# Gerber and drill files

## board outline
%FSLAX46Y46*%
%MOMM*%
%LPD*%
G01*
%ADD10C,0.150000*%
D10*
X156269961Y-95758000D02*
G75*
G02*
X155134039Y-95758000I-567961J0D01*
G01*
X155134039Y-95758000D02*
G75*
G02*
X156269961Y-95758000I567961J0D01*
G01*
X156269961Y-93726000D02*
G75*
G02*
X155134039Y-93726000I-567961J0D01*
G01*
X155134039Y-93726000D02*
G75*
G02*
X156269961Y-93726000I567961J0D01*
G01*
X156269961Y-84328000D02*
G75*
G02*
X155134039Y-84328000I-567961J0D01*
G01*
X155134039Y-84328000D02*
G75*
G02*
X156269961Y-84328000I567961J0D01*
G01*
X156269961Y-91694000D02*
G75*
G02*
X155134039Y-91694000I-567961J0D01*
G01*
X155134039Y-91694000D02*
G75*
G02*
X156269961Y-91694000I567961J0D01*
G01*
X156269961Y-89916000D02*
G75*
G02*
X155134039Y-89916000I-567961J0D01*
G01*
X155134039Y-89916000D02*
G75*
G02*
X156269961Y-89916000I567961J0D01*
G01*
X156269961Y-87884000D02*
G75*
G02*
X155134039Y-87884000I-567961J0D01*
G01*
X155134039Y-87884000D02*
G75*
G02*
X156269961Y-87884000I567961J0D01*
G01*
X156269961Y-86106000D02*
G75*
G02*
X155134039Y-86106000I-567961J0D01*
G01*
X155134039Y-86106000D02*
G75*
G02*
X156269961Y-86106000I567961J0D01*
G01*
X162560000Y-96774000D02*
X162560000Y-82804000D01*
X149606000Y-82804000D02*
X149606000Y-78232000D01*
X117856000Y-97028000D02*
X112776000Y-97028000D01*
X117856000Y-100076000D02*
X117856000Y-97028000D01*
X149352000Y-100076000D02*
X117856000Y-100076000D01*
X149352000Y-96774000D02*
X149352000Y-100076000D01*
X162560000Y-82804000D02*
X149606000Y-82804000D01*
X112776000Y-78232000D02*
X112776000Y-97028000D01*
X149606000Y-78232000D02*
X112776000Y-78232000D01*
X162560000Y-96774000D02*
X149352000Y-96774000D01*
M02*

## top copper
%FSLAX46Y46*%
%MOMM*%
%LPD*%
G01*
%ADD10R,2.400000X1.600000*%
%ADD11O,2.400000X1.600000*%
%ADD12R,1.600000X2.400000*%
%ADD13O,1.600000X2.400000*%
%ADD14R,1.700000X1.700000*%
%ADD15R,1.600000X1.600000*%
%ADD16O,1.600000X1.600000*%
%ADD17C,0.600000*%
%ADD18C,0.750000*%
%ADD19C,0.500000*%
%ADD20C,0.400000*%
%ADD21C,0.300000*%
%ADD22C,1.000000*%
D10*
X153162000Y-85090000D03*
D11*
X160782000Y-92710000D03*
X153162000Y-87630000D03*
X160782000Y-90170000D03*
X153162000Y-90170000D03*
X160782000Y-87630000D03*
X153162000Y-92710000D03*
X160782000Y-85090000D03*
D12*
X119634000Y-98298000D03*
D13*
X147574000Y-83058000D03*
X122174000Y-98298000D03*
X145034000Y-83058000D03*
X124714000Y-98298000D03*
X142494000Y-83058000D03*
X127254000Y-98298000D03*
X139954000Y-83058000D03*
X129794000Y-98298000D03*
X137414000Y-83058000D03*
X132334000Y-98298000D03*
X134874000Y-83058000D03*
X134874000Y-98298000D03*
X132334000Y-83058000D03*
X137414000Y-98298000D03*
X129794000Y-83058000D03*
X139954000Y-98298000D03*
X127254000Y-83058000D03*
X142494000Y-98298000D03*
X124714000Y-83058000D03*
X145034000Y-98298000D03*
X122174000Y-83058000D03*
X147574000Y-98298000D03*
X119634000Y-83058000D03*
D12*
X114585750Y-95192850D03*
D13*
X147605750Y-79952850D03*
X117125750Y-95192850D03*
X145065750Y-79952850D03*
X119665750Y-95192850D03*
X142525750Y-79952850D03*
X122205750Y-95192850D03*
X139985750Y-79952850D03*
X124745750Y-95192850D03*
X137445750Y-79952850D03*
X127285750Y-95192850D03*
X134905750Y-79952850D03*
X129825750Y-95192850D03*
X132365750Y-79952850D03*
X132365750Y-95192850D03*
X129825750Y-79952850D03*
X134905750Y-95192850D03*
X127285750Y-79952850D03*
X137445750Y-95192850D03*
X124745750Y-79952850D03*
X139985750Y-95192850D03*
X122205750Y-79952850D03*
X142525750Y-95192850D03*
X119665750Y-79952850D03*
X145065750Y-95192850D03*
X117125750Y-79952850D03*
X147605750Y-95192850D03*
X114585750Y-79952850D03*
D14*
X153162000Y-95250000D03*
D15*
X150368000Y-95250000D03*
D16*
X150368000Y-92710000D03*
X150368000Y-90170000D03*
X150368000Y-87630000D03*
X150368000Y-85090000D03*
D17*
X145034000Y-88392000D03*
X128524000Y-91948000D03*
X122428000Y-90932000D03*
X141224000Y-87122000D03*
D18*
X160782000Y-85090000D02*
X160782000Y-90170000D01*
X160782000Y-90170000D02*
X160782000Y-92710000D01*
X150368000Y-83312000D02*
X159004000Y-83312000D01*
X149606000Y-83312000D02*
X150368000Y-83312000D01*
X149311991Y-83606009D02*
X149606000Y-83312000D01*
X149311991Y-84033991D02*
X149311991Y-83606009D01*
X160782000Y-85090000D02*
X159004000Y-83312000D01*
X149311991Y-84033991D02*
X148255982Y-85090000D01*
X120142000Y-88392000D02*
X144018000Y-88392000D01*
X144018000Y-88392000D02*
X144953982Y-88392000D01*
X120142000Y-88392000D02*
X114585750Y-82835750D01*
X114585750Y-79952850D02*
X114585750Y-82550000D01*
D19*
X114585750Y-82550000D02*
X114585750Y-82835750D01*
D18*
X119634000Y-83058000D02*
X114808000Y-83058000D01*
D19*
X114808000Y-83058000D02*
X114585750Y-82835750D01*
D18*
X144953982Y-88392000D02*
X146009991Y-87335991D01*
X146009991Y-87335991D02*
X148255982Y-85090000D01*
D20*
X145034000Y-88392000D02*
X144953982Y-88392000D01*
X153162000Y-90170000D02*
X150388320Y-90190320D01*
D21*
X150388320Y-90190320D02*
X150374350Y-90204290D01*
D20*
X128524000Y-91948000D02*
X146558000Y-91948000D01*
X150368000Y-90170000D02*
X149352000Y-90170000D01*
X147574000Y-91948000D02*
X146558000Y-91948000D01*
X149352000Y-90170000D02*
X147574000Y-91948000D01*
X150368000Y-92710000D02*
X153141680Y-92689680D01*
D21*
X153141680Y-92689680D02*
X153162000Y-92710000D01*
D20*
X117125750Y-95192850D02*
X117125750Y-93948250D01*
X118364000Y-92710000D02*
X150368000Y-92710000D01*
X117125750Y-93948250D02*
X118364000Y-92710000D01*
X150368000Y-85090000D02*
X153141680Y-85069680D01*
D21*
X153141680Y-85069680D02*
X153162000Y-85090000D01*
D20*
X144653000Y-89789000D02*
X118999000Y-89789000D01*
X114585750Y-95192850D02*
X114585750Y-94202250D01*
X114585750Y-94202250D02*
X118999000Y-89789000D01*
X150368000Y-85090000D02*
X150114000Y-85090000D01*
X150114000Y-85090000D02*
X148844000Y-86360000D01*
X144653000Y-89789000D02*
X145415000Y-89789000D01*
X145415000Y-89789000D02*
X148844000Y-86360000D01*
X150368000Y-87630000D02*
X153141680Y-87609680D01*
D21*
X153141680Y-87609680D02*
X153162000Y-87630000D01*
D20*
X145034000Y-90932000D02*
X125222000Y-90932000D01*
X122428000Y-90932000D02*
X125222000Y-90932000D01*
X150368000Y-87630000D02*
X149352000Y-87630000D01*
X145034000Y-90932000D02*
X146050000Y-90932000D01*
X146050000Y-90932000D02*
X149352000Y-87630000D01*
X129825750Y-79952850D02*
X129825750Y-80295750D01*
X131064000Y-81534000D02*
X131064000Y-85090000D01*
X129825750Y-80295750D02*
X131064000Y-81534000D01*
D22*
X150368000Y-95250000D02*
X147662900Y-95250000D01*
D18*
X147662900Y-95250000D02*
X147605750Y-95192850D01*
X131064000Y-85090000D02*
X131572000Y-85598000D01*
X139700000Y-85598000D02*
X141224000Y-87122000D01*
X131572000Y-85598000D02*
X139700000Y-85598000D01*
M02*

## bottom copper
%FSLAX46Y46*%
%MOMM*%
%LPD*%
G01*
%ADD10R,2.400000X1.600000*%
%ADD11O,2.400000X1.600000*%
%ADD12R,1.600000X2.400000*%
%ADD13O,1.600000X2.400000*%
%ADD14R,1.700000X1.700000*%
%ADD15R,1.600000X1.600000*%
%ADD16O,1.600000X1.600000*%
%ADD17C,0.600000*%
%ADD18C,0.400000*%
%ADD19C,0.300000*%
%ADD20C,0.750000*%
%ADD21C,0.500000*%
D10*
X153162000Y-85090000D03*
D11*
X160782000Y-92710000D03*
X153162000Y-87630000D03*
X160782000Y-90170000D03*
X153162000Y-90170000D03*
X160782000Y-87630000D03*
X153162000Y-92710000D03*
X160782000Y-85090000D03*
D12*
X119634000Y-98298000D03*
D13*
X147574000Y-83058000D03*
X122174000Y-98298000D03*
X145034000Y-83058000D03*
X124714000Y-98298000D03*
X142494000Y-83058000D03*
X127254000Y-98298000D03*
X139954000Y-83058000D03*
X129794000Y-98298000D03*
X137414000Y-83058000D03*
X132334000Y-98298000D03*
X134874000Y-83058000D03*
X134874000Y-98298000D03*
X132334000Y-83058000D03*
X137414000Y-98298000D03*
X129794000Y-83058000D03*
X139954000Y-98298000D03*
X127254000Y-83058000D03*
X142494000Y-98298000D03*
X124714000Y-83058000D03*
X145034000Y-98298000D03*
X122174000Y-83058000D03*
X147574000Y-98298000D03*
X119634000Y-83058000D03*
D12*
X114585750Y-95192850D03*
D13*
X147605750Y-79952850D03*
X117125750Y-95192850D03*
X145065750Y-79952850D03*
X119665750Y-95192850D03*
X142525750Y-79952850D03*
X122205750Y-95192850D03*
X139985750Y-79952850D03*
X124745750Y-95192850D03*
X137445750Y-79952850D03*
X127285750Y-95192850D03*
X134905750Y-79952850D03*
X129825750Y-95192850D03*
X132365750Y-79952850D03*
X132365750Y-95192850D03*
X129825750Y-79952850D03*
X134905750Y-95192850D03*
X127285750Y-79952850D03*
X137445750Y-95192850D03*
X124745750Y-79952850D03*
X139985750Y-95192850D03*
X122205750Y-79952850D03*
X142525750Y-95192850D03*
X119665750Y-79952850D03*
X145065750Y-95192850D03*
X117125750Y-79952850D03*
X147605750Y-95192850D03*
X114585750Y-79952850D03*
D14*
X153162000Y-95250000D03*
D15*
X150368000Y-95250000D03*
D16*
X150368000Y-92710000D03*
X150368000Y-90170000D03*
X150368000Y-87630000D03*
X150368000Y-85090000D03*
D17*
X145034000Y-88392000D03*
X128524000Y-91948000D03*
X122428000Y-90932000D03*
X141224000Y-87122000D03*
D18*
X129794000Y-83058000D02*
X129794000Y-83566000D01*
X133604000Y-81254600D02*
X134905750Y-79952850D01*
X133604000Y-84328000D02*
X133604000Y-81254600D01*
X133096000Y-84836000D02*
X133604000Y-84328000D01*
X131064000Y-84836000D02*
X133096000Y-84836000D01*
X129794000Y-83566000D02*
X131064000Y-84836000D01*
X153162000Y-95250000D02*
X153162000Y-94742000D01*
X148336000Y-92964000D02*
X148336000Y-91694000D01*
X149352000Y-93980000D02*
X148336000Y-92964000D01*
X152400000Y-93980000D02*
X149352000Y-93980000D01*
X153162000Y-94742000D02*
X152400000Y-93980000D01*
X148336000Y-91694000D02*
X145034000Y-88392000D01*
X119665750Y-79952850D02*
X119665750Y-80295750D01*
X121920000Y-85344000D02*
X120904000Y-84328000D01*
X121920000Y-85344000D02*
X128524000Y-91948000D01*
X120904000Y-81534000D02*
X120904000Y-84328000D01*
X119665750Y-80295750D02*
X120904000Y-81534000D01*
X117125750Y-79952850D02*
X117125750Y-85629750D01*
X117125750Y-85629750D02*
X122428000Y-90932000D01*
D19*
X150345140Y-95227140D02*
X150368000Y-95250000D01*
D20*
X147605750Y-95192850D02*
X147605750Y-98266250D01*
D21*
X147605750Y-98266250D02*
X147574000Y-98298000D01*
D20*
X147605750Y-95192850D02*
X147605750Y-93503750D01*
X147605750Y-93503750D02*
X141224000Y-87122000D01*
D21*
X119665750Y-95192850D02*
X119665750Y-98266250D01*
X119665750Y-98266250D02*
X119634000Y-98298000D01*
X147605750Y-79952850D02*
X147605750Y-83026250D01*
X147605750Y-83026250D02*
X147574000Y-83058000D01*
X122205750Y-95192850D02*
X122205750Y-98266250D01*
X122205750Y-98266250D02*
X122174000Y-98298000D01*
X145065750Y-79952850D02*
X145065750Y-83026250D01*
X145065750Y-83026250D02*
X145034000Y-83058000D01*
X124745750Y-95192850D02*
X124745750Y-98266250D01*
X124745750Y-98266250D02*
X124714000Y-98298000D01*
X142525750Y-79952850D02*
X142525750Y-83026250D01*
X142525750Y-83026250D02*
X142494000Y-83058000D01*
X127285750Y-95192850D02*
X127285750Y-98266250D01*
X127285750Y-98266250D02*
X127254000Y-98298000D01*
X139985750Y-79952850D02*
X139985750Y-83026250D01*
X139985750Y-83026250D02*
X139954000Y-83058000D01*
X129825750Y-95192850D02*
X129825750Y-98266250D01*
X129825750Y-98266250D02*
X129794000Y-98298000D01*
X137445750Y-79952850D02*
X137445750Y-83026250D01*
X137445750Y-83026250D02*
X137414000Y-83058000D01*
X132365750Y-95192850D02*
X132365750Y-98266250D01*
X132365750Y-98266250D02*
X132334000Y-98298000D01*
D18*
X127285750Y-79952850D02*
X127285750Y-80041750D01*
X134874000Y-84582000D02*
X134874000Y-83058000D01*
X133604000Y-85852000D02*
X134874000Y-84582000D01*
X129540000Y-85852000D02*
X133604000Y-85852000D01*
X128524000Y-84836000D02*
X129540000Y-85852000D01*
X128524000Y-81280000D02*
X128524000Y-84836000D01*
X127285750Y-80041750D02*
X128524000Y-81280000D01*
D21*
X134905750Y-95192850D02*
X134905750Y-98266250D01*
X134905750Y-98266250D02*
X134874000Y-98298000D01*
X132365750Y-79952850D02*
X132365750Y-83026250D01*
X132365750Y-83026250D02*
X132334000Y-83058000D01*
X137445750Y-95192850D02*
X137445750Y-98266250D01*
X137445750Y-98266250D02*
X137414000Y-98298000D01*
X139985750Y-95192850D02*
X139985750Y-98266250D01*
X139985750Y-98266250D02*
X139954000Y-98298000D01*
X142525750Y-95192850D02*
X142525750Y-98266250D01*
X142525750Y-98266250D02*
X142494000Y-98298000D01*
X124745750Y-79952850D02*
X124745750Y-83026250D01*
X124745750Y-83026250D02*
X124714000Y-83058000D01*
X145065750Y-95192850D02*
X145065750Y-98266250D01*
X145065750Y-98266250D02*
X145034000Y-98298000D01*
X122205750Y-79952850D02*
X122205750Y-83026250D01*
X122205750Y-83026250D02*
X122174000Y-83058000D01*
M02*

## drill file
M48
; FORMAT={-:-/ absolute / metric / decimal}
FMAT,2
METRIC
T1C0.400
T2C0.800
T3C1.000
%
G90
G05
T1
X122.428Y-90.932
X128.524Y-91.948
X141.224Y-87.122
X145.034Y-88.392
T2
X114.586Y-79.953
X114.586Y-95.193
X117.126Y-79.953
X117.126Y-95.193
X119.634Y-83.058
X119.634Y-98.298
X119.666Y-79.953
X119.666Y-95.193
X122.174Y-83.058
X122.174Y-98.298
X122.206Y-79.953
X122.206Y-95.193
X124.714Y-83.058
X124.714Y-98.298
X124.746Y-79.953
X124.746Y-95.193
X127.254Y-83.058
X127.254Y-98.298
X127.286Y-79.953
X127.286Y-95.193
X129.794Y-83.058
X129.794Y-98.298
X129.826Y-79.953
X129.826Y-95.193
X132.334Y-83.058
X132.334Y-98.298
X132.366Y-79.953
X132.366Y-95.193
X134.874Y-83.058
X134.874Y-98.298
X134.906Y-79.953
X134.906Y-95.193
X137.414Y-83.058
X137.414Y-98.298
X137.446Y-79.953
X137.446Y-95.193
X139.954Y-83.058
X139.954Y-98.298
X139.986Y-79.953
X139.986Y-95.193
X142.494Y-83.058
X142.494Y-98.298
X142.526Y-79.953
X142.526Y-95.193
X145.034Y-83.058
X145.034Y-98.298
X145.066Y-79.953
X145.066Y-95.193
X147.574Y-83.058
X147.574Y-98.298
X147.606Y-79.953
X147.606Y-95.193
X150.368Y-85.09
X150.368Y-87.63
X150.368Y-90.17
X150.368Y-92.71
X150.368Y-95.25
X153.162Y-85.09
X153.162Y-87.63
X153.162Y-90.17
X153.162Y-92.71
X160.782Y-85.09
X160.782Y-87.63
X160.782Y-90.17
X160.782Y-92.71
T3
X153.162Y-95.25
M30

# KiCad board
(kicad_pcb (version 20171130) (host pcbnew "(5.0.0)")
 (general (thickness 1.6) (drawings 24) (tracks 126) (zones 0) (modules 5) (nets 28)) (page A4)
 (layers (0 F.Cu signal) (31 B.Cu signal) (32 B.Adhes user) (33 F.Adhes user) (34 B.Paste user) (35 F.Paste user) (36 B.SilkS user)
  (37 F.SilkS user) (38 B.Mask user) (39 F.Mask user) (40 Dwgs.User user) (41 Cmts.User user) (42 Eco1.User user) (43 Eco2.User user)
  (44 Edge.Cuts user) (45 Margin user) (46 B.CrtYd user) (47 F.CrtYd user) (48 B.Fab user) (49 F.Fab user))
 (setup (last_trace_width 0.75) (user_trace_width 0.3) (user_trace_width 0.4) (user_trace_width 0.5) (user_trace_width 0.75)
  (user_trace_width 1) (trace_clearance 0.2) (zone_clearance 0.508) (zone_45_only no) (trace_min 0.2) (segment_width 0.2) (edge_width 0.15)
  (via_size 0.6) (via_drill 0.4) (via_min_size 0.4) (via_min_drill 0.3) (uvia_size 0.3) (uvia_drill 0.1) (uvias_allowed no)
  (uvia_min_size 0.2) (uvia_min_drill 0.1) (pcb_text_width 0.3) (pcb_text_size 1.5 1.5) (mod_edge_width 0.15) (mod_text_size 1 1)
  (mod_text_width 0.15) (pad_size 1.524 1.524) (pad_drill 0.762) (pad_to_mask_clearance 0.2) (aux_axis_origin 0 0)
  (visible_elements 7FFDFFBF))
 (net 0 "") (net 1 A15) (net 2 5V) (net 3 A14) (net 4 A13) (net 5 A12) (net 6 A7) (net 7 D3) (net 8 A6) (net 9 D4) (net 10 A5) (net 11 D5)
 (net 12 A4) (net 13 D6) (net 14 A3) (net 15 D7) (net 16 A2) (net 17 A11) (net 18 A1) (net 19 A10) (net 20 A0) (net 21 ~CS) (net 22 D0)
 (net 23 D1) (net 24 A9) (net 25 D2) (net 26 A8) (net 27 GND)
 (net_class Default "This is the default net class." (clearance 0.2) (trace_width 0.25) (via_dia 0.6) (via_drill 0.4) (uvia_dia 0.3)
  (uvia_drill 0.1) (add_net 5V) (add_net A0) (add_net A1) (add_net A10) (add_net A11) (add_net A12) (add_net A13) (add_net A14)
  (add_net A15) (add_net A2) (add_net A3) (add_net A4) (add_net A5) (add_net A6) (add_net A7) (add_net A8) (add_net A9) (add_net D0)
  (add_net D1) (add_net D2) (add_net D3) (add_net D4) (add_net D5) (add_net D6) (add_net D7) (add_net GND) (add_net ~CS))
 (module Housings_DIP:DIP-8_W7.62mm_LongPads (layer F.Cu) (at 153.162 85.09)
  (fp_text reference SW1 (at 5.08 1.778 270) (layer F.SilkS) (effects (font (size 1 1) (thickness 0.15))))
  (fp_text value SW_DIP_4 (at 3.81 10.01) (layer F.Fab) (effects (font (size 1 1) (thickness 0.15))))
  (pad 1 thru_hole rect (at 0 0) (size 2.4 1.6) (drill 0.8) (layers *.Cu *.Mask) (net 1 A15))
  (pad 5 thru_hole oval (at 7.62 7.62) (size 2.4 1.6) (drill 0.8) (layers *.Cu *.Mask) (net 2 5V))
  (pad 2 thru_hole oval (at 0 2.54) (size 2.4 1.6) (drill 0.8) (layers *.Cu *.Mask) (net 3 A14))
  (pad 6 thru_hole oval (at 7.62 5.08) (size 2.4 1.6) (drill 0.8) (layers *.Cu *.Mask) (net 2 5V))
  (pad 3 thru_hole oval (at 0 5.08) (size 2.4 1.6) (drill 0.8) (layers *.Cu *.Mask) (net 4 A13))
  (pad 7 thru_hole oval (at 7.62 2.54) (size 2.4 1.6) (drill 0.8) (layers *.Cu *.Mask) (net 2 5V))
  (pad 4 thru_hole oval (at 0 7.62) (size 2.4 1.6) (drill 0.8) (layers *.Cu *.Mask) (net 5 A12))
  (pad 8 thru_hole oval (at 7.62 0) (size 2.4 1.6) (drill 0.8) (layers *.Cu *.Mask) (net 2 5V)))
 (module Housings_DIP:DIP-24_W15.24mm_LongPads (layer F.Cu) (at 119.634 98.298 90)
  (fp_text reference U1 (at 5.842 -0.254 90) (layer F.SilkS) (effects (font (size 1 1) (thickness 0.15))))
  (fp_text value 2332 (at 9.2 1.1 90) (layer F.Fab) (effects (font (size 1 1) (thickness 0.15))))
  (pad 1 thru_hole rect (at 0 0 90) (size 2.4 1.6) (drill 0.8) (layers *.Cu *.Mask) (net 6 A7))
  (pad 13 thru_hole oval (at 15.24 27.94 90) (size 2.4 1.6) (drill 0.8) (layers *.Cu *.Mask) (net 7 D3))
  (pad 2 thru_hole oval (at 0 2.54 90) (size 2.4 1.6) (drill 0.8) (layers *.Cu *.Mask) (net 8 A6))
  (pad 14 thru_hole oval (at 15.24 25.4 90) (size 2.4 1.6) (drill 0.8) (layers *.Cu *.Mask) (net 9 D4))
  (pad 3 thru_hole oval (at 0 5.08 90) (size 2.4 1.6) (drill 0.8) (layers *.Cu *.Mask) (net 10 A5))
  (pad 15 thru_hole oval (at 15.24 22.86 90) (size 2.4 1.6) (drill 0.8) (layers *.Cu *.Mask) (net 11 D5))
  (pad 4 thru_hole oval (at 0 7.62 90) (size 2.4 1.6) (drill 0.8) (layers *.Cu *.Mask) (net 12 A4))
  (pad 16 thru_hole oval (at 15.24 20.32 90) (size 2.4 1.6) (drill 0.8) (layers *.Cu *.Mask) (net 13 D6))
  (pad 5 thru_hole oval (at 0 10.16 90) (size 2.4 1.6) (drill 0.8) (layers *.Cu *.Mask) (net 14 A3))
  (pad 17 thru_hole oval (at 15.24 17.78 90) (size 2.4 1.6) (drill 0.8) (layers *.Cu *.Mask) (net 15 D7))
  (pad 6 thru_hole oval (at 0 12.7 90) (size 2.4 1.6) (drill 0.8) (layers *.Cu *.Mask) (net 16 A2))
  (pad 18 thru_hole oval (at 15.24 15.24 90) (size 2.4 1.6) (drill 0.8) (layers *.Cu *.Mask) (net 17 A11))
  (pad 7 thru_hole oval (at 0 15.24 90) (size 2.4 1.6) (drill 0.8) (layers *.Cu *.Mask) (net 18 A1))
  (pad 19 thru_hole oval (at 15.24 12.7 90) (size 2.4 1.6) (drill 0.8) (layers *.Cu *.Mask) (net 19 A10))
  (pad 8 thru_hole oval (at 0 17.78 90) (size 2.4 1.6) (drill 0.8) (layers *.Cu *.Mask) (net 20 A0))
  (pad 20 thru_hole oval (at 15.24 10.16 90) (size 2.4 1.6) (drill 0.8) (layers *.Cu *.Mask) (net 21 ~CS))
  (pad 9 thru_hole oval (at 0 20.32 90) (size 2.4 1.6) (drill 0.8) (layers *.Cu *.Mask) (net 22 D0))
  (pad 21 thru_hole oval (at 15.24 7.62 90) (size 2.4 1.6) (drill 0.8) (layers *.Cu *.Mask))
  (pad 10 thru_hole oval (at 0 22.86 90) (size 2.4 1.6) (drill 0.8) (layers *.Cu *.Mask) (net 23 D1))
  (pad 22 thru_hole oval (at 15.24 5.08 90) (size 2.4 1.6) (drill 0.8) (layers *.Cu *.Mask) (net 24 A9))
  (pad 11 thru_hole oval (at 0 25.4 90) (size 2.4 1.6) (drill 0.8) (layers *.Cu *.Mask) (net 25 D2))
  (pad 23 thru_hole oval (at 15.24 2.54 90) (size 2.4 1.6) (drill 0.8) (layers *.Cu *.Mask) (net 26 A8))
  (pad 12 thru_hole oval (at 0 27.94 90) (size 2.4 1.6) (drill 0.8) (layers *.Cu *.Mask) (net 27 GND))
  (pad 24 thru_hole oval (at 15.24 0 90) (size 2.4 1.6) (drill 0.8) (layers *.Cu *.Mask) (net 2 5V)))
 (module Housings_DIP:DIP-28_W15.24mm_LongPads (layer F.Cu) (at 114.58575 95.19285 90)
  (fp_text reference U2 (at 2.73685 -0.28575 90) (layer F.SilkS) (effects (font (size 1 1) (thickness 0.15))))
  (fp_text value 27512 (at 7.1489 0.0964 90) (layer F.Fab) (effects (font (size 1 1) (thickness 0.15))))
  (pad 1 thru_hole rect (at 0 0 90) (size 2.4 1.6) (drill 0.8) (layers *.Cu *.Mask) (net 1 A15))
  (pad 15 thru_hole oval (at 15.24 33.02 90) (size 2.4 1.6) (drill 0.8) (layers *.Cu *.Mask) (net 7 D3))
  (pad 2 thru_hole oval (at 0 2.54 90) (size 2.4 1.6) (drill 0.8) (layers *.Cu *.Mask) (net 5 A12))
  (pad 16 thru_hole oval (at 15.24 30.48 90) (size 2.4 1.6) (drill 0.8) (layers *.Cu *.Mask) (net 9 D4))
  (pad 3 thru_hole oval (at 0 5.08 90) (size 2.4 1.6) (drill 0.8) (layers *.Cu *.Mask) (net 6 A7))
  (pad 17 thru_hole oval (at 15.24 27.94 90) (size 2.4 1.6) (drill 0.8) (layers *.Cu *.Mask) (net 11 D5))
  (pad 4 thru_hole oval (at 0 7.62 90) (size 2.4 1.6) (drill 0.8) (layers *.Cu *.Mask) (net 8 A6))
  (pad 18 thru_hole oval (at 15.24 25.4 90) (size 2.4 1.6) (drill 0.8) (layers *.Cu *.Mask) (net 13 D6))
  (pad 5 thru_hole oval (at 0 10.16 90) (size 2.4 1.6) (drill 0.8) (layers *.Cu *.Mask) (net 10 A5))
  (pad 19 thru_hole oval (at 15.24 22.86 90) (size 2.4 1.6) (drill 0.8) (layers *.Cu *.Mask) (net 15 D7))
  (pad 6 thru_hole oval (at 0 12.7 90) (size 2.4 1.6) (drill 0.8) (layers *.Cu *.Mask) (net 12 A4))
  (pad 20 thru_hole oval (at 15.24 20.32 90) (size 2.4 1.6) (drill 0.8) (layers *.Cu *.Mask) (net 21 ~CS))
  (pad 7 thru_hole oval (at 0 15.24 90) (size 2.4 1.6) (drill 0.8) (layers *.Cu *.Mask) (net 14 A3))
  (pad 21 thru_hole oval (at 15.24 17.78 90) (size 2.4 1.6) (drill 0.8) (layers *.Cu *.Mask) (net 19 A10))
  (pad 8 thru_hole oval (at 0 17.78 90) (size 2.4 1.6) (drill 0.8) (layers *.Cu *.Mask) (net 16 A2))
  (pad 22 thru_hole oval (at 15.24 15.24 90) (size 2.4 1.6) (drill 0.8) (layers *.Cu *.Mask) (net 27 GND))
  (pad 9 thru_hole oval (at 0 20.32 90) (size 2.4 1.6) (drill 0.8) (layers *.Cu *.Mask) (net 18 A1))
  (pad 23 thru_hole oval (at 15.24 12.7 90) (size 2.4 1.6) (drill 0.8) (layers *.Cu *.Mask) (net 17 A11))
  (pad 10 thru_hole oval (at 0 22.86 90) (size 2.4 1.6) (drill 0.8) (layers *.Cu *.Mask) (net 20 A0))
  (pad 24 thru_hole oval (at 15.24 10.16 90) (size 2.4 1.6) (drill 0.8) (layers *.Cu *.Mask) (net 24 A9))
  (pad 11 thru_hole oval (at 0 25.4 90) (size 2.4 1.6) (drill 0.8) (layers *.Cu *.Mask) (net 22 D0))
  (pad 25 thru_hole oval (at 15.24 7.62 90) (size 2.4 1.6) (drill 0.8) (layers *.Cu *.Mask) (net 26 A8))
  (pad 12 thru_hole oval (at 0 27.94 90) (size 2.4 1.6) (drill 0.8) (layers *.Cu *.Mask) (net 23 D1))
  (pad 26 thru_hole oval (at 15.24 5.08 90) (size 2.4 1.6) (drill 0.8) (layers *.Cu *.Mask) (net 4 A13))
  (pad 13 thru_hole oval (at 0 30.48 90) (size 2.4 1.6) (drill 0.8) (layers *.Cu *.Mask) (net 25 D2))
  (pad 27 thru_hole oval (at 15.24 2.54 90) (size 2.4 1.6) (drill 0.8) (layers *.Cu *.Mask) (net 3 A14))
  (pad 14 thru_hole oval (at 0 33.02 90) (size 2.4 1.6) (drill 0.8) (layers *.Cu *.Mask) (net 27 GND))
  (pad 28 thru_hole oval (at 15.24 0 90) (size 2.4 1.6) (drill 0.8) (layers *.Cu *.Mask) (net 2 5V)))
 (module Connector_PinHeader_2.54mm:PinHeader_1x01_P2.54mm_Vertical (layer F.Cu) (at 153.162 95.25 90)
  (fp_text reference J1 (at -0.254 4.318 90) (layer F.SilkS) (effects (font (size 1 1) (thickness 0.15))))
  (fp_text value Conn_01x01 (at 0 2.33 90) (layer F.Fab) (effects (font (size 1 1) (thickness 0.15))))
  (pad 1 thru_hole rect (at 0 0 90) (size 1.7 1.7) (drill 1) (layers *.Cu *.Mask) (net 2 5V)))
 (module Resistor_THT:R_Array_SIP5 (layer F.Cu) (at 150.368 95.25 90)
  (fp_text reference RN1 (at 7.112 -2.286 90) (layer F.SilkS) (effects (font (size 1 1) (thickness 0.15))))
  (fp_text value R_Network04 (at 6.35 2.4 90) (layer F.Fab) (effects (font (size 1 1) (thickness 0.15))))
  (pad 1 thru_hole rect (at 0 0 90) (size 1.6 1.6) (drill 0.8) (layers *.Cu *.Mask) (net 27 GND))
  (pad 2 thru_hole oval (at 2.54 0 90) (size 1.6 1.6) (drill 0.8) (layers *.Cu *.Mask) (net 5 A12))
  (pad 3 thru_hole oval (at 5.08 0 90) (size 1.6 1.6) (drill 0.8) (layers *.Cu *.Mask) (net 4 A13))
  (pad 4 thru_hole oval (at 7.62 0 90) (size 1.6 1.6) (drill 0.8) (layers *.Cu *.Mask) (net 3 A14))
  (pad 5 thru_hole oval (at 10.16 0 90) (size 1.6 1.6) (drill 0.8) (layers *.Cu *.Mask) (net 1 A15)))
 (gr_circle (center 155.702 95.758) (end 156.21 96.012) (layer Edge.Cuts) (width 0.15))
 (gr_circle (center 155.702 93.726) (end 156.21 93.98) (layer Edge.Cuts) (width 0.15))
 (gr_circle (center 155.702 84.328) (end 156.21 84.582) (layer Edge.Cuts) (width 0.15))
 (gr_circle (center 155.702 91.694) (end 155.956 92.202) (layer Edge.Cuts) (width 0.15))
 (gr_circle (center 155.702 89.916) (end 156.21 90.17) (layer Edge.Cuts) (width 0.15))
 (gr_circle (center 155.702 87.884) (end 156.21 88.138) (layer Edge.Cuts) (width 0.15))
 (gr_circle (center 155.702 86.106) (end 156.21 86.36) (layer Edge.Cuts) (width 0.15))
 (gr_line (start 162.56 96.774) (end 162.56 82.804) (angle 90) (layer Edge.Cuts) (width 0.15))
 (gr_line (start 149.606 82.804) (end 149.606 78.232) (angle 90) (layer Edge.Cuts) (width 0.15))
 (gr_line (start 117.856 97.028) (end 112.776 97.028) (angle 90) (layer Edge.Cuts) (width 0.15))
 (gr_line (start 117.856 100.076) (end 117.856 97.028) (angle 90) (layer Edge.Cuts) (width 0.15))
 (gr_line (start 149.352 100.076) (end 117.856 100.076) (angle 90) (layer Edge.Cuts) (width 0.15))
 (gr_line (start 149.352 96.774) (end 149.352 100.076) (angle 90) (layer Edge.Cuts) (width 0.15))
 (gr_line (start 162.56 82.804) (end 149.606 82.804) (angle 90) (layer Edge.Cuts) (width 0.15))
 (gr_line (start 112.776 78.232) (end 112.776 97.028) (angle 90) (layer Edge.Cuts) (width 0.15))
 (gr_line (start 149.606 78.232) (end 112.776 78.232) (angle 90) (layer Edge.Cuts) (width 0.15))
 (gr_line (start 162.56 96.774) (end 149.352 96.774) (angle 90) (layer Edge.Cuts) (width 0.15))
 (segment (start 129.794 83.058) (end 129.794 83.566) (width 0.4) (layer B.Cu) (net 21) (status C00000))
 (segment (start 133.604 81.2546) (end 134.90575 79.95285) (width 0.4) (layer B.Cu) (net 21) (status 800000))
 (segment (start 133.604 84.328) (end 133.604 81.2546) (width 0.4) (layer B.Cu) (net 21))
 (segment (start 133.096 84.836) (end 133.604 84.328) (width 0.4) (layer B.Cu) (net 21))
 (segment (start 131.064 84.836) (end 133.096 84.836) (width 0.4) (layer B.Cu) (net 21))
 (segment (start 129.794 83.566) (end 131.064 84.836) (width 0.4) (layer B.Cu) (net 21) (status 400000))
 (segment (start 160.782 85.09) (end 160.782 90.17) (width 0.75) (layer F.Cu) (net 2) (status C00030))
 (segment (start 160.782 90.17) (end 160.782 92.71) (width 0.75) (layer F.Cu) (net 2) (status C00030))
 (segment (start 150.368 83.312) (end 159.004 83.312) (width 0.75) (layer F.Cu) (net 2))
 (segment (start 149.606 83.312) (end 150.368 83.312) (width 0.75) (layer F.Cu) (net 2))
 (segment (start 149.311991 83.606009) (end 149.606 83.312) (width 0.75) (layer F.Cu) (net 2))
 (segment (start 149.311991 84.033991) (end 149.311991 83.606009) (width 0.75) (layer F.Cu) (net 2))
 (segment (start 160.782 85.09) (end 159.004 83.312) (width 0.75) (layer F.Cu) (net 2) (status 400000))
 (segment (start 149.311991 84.033991) (end 148.255982 85.09) (width 0.75) (layer F.Cu) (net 2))
 (segment (start 120.142 88.392) (end 144.018 88.392) (width 0.75) (layer F.Cu) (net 2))
 (segment (start 144.018 88.392) (end 144.953982 88.392) (width 0.75) (layer F.Cu) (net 2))
 (segment (start 120.142 88.392) (end 114.58575 82.83575) (width 0.75) (layer F.Cu) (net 2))
 (segment (start 114.58575 79.95285) (end 114.58575 82.55) (width 0.75) (layer F.Cu) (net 2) (status 400000))
 (segment (start 114.58575 82.55) (end 114.58575 82.83575) (width 0.5) (layer F.Cu) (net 2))
 (segment (start 119.634 83.058) (end 114.808 83.058) (width 0.75) (layer F.Cu) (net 2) (status 400000))
 (segment (start 114.808 83.058) (end 114.58575 82.83575) (width 0.5) (layer F.Cu) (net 2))
 (segment (start 144.953982 88.392) (end 146.009991 87.335991) (width 0.75) (layer F.Cu) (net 2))
 (segment (start 146.009991 87.335991) (end 148.255982 85.09) (width 0.75) (layer F.Cu) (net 2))
 (segment (start 153.162 95.25) (end 153.162 94.742) (width 0.4) (layer B.Cu) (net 2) (status C00000))
 (segment (start 148.336 92.964) (end 148.336 91.694) (width 0.4) (layer B.Cu) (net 2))
 (segment (start 149.352 93.98) (end 148.336 92.964) (width 0.4) (layer B.Cu) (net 2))
 (segment (start 152.4 93.98) (end 149.352 93.98) (width 0.4) (layer B.Cu) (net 2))
 (segment (start 153.162 94.742) (end 152.4 93.98) (width 0.4) (layer B.Cu) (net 2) (status 400000))
 (segment (start 148.336 91.694) (end 145.034 88.392) (width 0.4) (layer B.Cu) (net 2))
 (segment (start 145.034 88.392) (end 144.953982 88.392) (width 0.4) (layer F.Cu) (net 2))
 (via (at 145.034 88.392) (size 0.6) (drill 0.4) (layers F.Cu B.Cu) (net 2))
 (segment (start 153.162 90.17) (end 150.38832 90.19032) (width 0.4) (layer F.Cu) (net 4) (status C00010))
 (segment (start 150.38832 90.19032) (end 150.37435 90.20429) (width 0.3) (layer F.Cu) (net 4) (status C00030))
 (segment (start 119.66575 79.95285) (end 119.66575 80.29575) (width 0.4) (layer B.Cu) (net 4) (status C00000))
 (segment (start 121.92 85.344) (end 120.904 84.328) (width 0.4) (layer B.Cu) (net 4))
 (segment (start 121.92 85.344) (end 128.524 91.948) (width 0.4) (layer B.Cu) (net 4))
 (via (at 128.524 91.948) (size 0.6) (drill 0.4) (layers F.Cu B.Cu) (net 4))
 (segment (start 128.524 91.948) (end 146.558 91.948) (width 0.4) (layer F.Cu) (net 4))
 (segment (start 120.904 81.534) (end 120.904 84.328) (width 0.4) (layer B.Cu) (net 4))
 (segment (start 119.66575 80.29575) (end 120.904 81.534) (width 0.4) (layer B.Cu) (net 4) (status 400000))
 (segment (start 150.368 90.17) (end 149.352 90.17) (width 0.4) (layer F.Cu) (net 4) (status 400000))
 (segment (start 147.574 91.948) (end 146.558 91.948) (width 0.4) (layer F.Cu) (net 4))
 (segment (start 149.352 90.17) (end 147.574 91.948) (width 0.4) (layer F.Cu) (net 4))
 (segment (start 150.368 92.71) (end 153.14168 92.68968) (width 0.4) (layer F.Cu) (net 5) (status C00020))
 (segment (start 153.14168 92.68968) (end 153.162 92.71) (width 0.3) (layer F.Cu) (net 5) (status C00030))
 (segment (start 117.12575 95.19285) (end 117.12575 93.94825) (width 0.4) (layer F.Cu) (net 5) (status 400000))
 (segment (start 118.364 92.71) (end 150.368 92.71) (width 0.4) (layer F.Cu) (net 5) (status 800000))
 (segment (start 117.12575 93.94825) (end 118.364 92.71) (width 0.4) (layer F.Cu) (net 5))
 (segment (start 150.368 85.09) (end 153.14168 85.06968) (width 0.4) (layer F.Cu) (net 1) (status C00020))
 (segment (start 153.14168 85.06968) (end 153.162 85.09) (width 0.3) (layer F.Cu) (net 1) (status C00030))
 (segment (start 144.653 89.789) (end 118.999 89.789) (width 0.4) (layer F.Cu) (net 1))
 (segment (start 114.58575 95.19285) (end 114.58575 94.20225) (width 0.4) (layer F.Cu) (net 1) (status C00000))
 (segment (start 114.58575 94.20225) (end 118.999 89.789) (width 0.4) (layer F.Cu) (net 1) (status 400000))
 (segment (start 150.368 85.09) (end 150.114 85.09) (width 0.4) (layer F.Cu) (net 1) (status C00000))
 (segment (start 150.114 85.09) (end 148.844 86.36) (width 0.4) (layer F.Cu) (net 1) (status 400000))
 (segment (start 144.653 89.789) (end 145.415 89.789) (width 0.4) (layer F.Cu) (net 1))
 (segment (start 145.415 89.789) (end 148.844 86.36) (width 0.4) (layer F.Cu) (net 1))
 (segment (start 150.368 87.63) (end 153.14168 87.60968) (width 0.4) (layer F.Cu) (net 3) (status C00020))
 (segment (start 153.14168 87.60968) (end 153.162 87.63) (width 0.3) (layer F.Cu) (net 3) (status C00030))
 (segment (start 145.034 90.932) (end 125.222 90.932) (width 0.4) (layer F.Cu) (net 3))
 (segment (start 117.12575 79.95285) (end 117.12575 85.62975) (width 0.4) (layer B.Cu) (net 3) (status 400000))
 (segment (start 122.428 90.932) (end 125.222 90.932) (width 0.4) (layer F.Cu) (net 3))
 (via (at 122.428 90.932) (size 0.6) (drill 0.4) (layers F.Cu B.Cu) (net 3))
 (segment (start 117.12575 85.62975) (end 122.428 90.932) (width 0.4) (layer B.Cu) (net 3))
 (segment (start 150.368 87.63) (end 149.352 87.63) (width 0.4) (layer F.Cu) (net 3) (status 400000))
 (segment (start 145.034 90.932) (end 146.05 90.932) (width 0.4) (layer F.Cu) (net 3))
 (segment (start 146.05 90.932) (end 149.352 87.63) (width 0.4) (layer F.Cu) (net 3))
 (segment (start 150.34514 95.22714) (end 150.368 95.25) (width 0.3) (layer B.Cu) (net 27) (status C00030))
 (segment (start 147.60575 95.19285) (end 147.60575 98.26625) (width 0.75) (layer B.Cu) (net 27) (status C00000))
 (segment (start 147.60575 98.26625) (end 147.574 98.298) (width 0.5) (layer B.Cu) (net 27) (status C00000))
 (segment (start 129.82575 79.95285) (end 129.82575 80.29575) (width 0.4) (layer F.Cu) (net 27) (status C00000))
 (segment (start 131.064 81.534) (end 131.064 85.09) (width 0.4) (layer F.Cu) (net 27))
 (segment (start 129.82575 80.29575) (end 131.064 81.534) (width 0.4) (layer F.Cu) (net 27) (status 400000))
 (segment (start 150.368 95.25) (end 147.6629 95.25) (width 1) (layer F.Cu) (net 27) (status C00000))
 (segment (start 147.6629 95.25) (end 147.60575 95.19285) (width 0.75) (layer F.Cu) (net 27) (status C00000))
 (segment (start 147.60575 95.19285) (end 147.60575 93.50375) (width 0.75) (layer B.Cu) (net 27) (status 400000))
 (via (at 141.224 87.122) (size 0.6) (drill 0.4) (layers F.Cu B.Cu) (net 27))
 (segment (start 147.60575 93.50375) (end 141.224 87.122) (width 0.75) (layer B.Cu) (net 27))
 (segment (start 131.064 85.09) (end 131.572 85.598) (width 0.75) (layer F.Cu) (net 27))
 (segment (start 139.7 85.598) (end 141.224 87.122) (width 0.75) (layer F.Cu) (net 27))
 (segment (start 131.572 85.598) (end 139.7 85.598) (width 0.75) (layer F.Cu) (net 27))
 (segment (start 119.66575 95.19285) (end 119.66575 98.26625) (width 0.5) (layer B.Cu) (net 6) (status C00000))
 (segment (start 119.66575 98.26625) (end 119.634 98.298) (width 0.5) (layer B.Cu) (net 6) (status C00000))
 (segment (start 147.60575 79.95285) (end 147.60575 83.02625) (width 0.5) (layer B.Cu) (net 7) (status C00000))
 (segment (start 147.60575 83.02625) (end 147.574 83.058) (width 0.5) (layer B.Cu) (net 7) (status C00000))
 (segment (start 122.20575 95.19285) (end 122.20575 98.26625) (width 0.5) (layer B.Cu) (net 8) (status C00000))
 (segment (start 122.20575 98.26625) (end 122.174 98.298) (width 0.5) (layer B.Cu) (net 8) (status C00000))
 (segment (start 145.06575 79.95285) (end 145.06575 83.02625) (width 0.5) (layer B.Cu) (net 9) (status C00000))
 (segment (start 145.06575 83.02625) (end 145.034 83.058) (width 0.5) (layer B.Cu) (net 9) (status C00000))
 (segment (start 124.74575 95.19285) (end 124.74575 98.26625) (width 0.5) (layer B.Cu) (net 10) (status C00000))
 (segment (start 124.74575 98.26625) (end 124.714 98.298) (width 0.5) (layer B.Cu) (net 10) (status C00000))
 (segment (start 142.52575 79.95285) (end 142.52575 83.02625) (width 0.5) (layer B.Cu) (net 11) (status C00000))
 (segment (start 142.52575 83.02625) (end 142.494 83.058) (width 0.5) (layer B.Cu) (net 11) (status C00000))
 (segment (start 127.28575 95.19285) (end 127.28575 98.26625) (width 0.5) (layer B.Cu) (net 12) (status C00000))
 (segment (start 127.28575 98.26625) (end 127.254 98.298) (width 0.5) (layer B.Cu) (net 12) (status C00000))
 (segment (start 139.98575 79.95285) (end 139.98575 83.02625) (width 0.5) (layer B.Cu) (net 13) (status C00000))
 (segment (start 139.98575 83.02625) (end 139.954 83.058) (width 0.5) (layer B.Cu) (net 13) (status C00000))
 (segment (start 129.82575 95.19285) (end 129.82575 98.26625) (width 0.5) (layer B.Cu) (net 14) (status C00000))
 (segment (start 129.82575 98.26625) (end 129.794 98.298) (width 0.5) (layer B.Cu) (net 14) (status C00000))
 (segment (start 137.44575 79.95285) (end 137.44575 83.02625) (width 0.5) (layer B.Cu) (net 15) (status C00000))
 (segment (start 137.44575 83.02625) (end 137.414 83.058) (width 0.5) (layer B.Cu) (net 15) (status C00000))
 (segment (start 132.36575 95.19285) (end 132.36575 98.26625) (width 0.5) (layer B.Cu) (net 16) (status C00000))
 (segment (start 132.36575 98.26625) (end 132.334 98.298) (width 0.5) (layer B.Cu) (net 16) (status C00000))
 (segment (start 127.28575 79.95285) (end 127.28575 80.04175) (width 0.4) (layer B.Cu) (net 17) (status C00000))
 (segment (start 134.874 84.582) (end 134.874 83.058) (width 0.4) (layer B.Cu) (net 17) (status 800000))
 (segment (start 133.604 85.852) (end 134.874 84.582) (width 0.4) (layer B.Cu) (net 17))
 (segment (start 129.54 85.852) (end 133.604 85.852) (width 0.4) (layer B.Cu) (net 17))
 (segment (start 128.524 84.836) (end 129.54 85.852) (width 0.4) (layer B.Cu) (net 17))
 (segment (start 128.524 81.28) (end 128.524 84.836) (width 0.4) (layer B.Cu) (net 17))
 (segment (start 127.28575 80.04175) (end 128.524 81.28) (width 0.4) (layer B.Cu) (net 17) (status 400000))
 (segment (start 134.90575 95.19285) (end 134.90575 98.26625) (width 0.5) (layer B.Cu) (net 18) (status C00000))
 (segment (start 134.90575 98.26625) (end 134.874 98.298) (width 0.5) (layer B.Cu) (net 18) (status C00000))
 (segment (start 132.36575 79.95285) (end 132.36575 83.02625) (width 0.5) (layer B.Cu) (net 19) (status C00000))
 (segment (start 132.36575 83.02625) (end 132.334 83.058) (width 0.5) (layer B.Cu) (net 19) (status C00000))
 (segment (start 137.44575 95.19285) (end 137.44575 98.26625) (width 0.5) (layer B.Cu) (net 20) (status C00000))
 (segment (start 137.44575 98.26625) (end 137.414 98.298) (width 0.5) (layer B.Cu) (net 20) (status C00000))
 (segment (start 139.98575 95.19285) (end 139.98575 98.26625) (width 0.5) (layer B.Cu) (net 22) (status C00000))
 (segment (start 139.98575 98.26625) (end 139.954 98.298) (width 0.5) (layer B.Cu) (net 22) (status C00000))
 (segment (start 142.52575 95.19285) (end 142.52575 98.26625) (width 0.5) (layer B.Cu) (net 23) (status C00000))
 (segment (start 142.52575 98.26625) (end 142.494 98.298) (width 0.5) (layer B.Cu) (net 23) (status C00000))
 (segment (start 124.74575 79.95285) (end 124.74575 83.02625) (width 0.5) (layer B.Cu) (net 24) (status C00000))
 (segment (start 124.74575 83.02625) (end 124.714 83.058) (width 0.5) (layer B.Cu) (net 24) (status C00000))
 (segment (start 145.06575 95.19285) (end 145.06575 98.26625) (width 0.5) (layer B.Cu) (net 25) (status C00000))
 (segment (start 145.06575 98.26625) (end 145.034 98.298) (width 0.5) (layer B.Cu) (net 25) (status C00000))
 (segment (start 122.20575 79.95285) (end 122.20575 83.02625) (width 0.5) (layer B.Cu) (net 26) (status C00000))
 (segment (start 122.20575 83.02625) (end 122.174 83.058) (width 0.5) (layer B.Cu) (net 26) (status C00000)))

